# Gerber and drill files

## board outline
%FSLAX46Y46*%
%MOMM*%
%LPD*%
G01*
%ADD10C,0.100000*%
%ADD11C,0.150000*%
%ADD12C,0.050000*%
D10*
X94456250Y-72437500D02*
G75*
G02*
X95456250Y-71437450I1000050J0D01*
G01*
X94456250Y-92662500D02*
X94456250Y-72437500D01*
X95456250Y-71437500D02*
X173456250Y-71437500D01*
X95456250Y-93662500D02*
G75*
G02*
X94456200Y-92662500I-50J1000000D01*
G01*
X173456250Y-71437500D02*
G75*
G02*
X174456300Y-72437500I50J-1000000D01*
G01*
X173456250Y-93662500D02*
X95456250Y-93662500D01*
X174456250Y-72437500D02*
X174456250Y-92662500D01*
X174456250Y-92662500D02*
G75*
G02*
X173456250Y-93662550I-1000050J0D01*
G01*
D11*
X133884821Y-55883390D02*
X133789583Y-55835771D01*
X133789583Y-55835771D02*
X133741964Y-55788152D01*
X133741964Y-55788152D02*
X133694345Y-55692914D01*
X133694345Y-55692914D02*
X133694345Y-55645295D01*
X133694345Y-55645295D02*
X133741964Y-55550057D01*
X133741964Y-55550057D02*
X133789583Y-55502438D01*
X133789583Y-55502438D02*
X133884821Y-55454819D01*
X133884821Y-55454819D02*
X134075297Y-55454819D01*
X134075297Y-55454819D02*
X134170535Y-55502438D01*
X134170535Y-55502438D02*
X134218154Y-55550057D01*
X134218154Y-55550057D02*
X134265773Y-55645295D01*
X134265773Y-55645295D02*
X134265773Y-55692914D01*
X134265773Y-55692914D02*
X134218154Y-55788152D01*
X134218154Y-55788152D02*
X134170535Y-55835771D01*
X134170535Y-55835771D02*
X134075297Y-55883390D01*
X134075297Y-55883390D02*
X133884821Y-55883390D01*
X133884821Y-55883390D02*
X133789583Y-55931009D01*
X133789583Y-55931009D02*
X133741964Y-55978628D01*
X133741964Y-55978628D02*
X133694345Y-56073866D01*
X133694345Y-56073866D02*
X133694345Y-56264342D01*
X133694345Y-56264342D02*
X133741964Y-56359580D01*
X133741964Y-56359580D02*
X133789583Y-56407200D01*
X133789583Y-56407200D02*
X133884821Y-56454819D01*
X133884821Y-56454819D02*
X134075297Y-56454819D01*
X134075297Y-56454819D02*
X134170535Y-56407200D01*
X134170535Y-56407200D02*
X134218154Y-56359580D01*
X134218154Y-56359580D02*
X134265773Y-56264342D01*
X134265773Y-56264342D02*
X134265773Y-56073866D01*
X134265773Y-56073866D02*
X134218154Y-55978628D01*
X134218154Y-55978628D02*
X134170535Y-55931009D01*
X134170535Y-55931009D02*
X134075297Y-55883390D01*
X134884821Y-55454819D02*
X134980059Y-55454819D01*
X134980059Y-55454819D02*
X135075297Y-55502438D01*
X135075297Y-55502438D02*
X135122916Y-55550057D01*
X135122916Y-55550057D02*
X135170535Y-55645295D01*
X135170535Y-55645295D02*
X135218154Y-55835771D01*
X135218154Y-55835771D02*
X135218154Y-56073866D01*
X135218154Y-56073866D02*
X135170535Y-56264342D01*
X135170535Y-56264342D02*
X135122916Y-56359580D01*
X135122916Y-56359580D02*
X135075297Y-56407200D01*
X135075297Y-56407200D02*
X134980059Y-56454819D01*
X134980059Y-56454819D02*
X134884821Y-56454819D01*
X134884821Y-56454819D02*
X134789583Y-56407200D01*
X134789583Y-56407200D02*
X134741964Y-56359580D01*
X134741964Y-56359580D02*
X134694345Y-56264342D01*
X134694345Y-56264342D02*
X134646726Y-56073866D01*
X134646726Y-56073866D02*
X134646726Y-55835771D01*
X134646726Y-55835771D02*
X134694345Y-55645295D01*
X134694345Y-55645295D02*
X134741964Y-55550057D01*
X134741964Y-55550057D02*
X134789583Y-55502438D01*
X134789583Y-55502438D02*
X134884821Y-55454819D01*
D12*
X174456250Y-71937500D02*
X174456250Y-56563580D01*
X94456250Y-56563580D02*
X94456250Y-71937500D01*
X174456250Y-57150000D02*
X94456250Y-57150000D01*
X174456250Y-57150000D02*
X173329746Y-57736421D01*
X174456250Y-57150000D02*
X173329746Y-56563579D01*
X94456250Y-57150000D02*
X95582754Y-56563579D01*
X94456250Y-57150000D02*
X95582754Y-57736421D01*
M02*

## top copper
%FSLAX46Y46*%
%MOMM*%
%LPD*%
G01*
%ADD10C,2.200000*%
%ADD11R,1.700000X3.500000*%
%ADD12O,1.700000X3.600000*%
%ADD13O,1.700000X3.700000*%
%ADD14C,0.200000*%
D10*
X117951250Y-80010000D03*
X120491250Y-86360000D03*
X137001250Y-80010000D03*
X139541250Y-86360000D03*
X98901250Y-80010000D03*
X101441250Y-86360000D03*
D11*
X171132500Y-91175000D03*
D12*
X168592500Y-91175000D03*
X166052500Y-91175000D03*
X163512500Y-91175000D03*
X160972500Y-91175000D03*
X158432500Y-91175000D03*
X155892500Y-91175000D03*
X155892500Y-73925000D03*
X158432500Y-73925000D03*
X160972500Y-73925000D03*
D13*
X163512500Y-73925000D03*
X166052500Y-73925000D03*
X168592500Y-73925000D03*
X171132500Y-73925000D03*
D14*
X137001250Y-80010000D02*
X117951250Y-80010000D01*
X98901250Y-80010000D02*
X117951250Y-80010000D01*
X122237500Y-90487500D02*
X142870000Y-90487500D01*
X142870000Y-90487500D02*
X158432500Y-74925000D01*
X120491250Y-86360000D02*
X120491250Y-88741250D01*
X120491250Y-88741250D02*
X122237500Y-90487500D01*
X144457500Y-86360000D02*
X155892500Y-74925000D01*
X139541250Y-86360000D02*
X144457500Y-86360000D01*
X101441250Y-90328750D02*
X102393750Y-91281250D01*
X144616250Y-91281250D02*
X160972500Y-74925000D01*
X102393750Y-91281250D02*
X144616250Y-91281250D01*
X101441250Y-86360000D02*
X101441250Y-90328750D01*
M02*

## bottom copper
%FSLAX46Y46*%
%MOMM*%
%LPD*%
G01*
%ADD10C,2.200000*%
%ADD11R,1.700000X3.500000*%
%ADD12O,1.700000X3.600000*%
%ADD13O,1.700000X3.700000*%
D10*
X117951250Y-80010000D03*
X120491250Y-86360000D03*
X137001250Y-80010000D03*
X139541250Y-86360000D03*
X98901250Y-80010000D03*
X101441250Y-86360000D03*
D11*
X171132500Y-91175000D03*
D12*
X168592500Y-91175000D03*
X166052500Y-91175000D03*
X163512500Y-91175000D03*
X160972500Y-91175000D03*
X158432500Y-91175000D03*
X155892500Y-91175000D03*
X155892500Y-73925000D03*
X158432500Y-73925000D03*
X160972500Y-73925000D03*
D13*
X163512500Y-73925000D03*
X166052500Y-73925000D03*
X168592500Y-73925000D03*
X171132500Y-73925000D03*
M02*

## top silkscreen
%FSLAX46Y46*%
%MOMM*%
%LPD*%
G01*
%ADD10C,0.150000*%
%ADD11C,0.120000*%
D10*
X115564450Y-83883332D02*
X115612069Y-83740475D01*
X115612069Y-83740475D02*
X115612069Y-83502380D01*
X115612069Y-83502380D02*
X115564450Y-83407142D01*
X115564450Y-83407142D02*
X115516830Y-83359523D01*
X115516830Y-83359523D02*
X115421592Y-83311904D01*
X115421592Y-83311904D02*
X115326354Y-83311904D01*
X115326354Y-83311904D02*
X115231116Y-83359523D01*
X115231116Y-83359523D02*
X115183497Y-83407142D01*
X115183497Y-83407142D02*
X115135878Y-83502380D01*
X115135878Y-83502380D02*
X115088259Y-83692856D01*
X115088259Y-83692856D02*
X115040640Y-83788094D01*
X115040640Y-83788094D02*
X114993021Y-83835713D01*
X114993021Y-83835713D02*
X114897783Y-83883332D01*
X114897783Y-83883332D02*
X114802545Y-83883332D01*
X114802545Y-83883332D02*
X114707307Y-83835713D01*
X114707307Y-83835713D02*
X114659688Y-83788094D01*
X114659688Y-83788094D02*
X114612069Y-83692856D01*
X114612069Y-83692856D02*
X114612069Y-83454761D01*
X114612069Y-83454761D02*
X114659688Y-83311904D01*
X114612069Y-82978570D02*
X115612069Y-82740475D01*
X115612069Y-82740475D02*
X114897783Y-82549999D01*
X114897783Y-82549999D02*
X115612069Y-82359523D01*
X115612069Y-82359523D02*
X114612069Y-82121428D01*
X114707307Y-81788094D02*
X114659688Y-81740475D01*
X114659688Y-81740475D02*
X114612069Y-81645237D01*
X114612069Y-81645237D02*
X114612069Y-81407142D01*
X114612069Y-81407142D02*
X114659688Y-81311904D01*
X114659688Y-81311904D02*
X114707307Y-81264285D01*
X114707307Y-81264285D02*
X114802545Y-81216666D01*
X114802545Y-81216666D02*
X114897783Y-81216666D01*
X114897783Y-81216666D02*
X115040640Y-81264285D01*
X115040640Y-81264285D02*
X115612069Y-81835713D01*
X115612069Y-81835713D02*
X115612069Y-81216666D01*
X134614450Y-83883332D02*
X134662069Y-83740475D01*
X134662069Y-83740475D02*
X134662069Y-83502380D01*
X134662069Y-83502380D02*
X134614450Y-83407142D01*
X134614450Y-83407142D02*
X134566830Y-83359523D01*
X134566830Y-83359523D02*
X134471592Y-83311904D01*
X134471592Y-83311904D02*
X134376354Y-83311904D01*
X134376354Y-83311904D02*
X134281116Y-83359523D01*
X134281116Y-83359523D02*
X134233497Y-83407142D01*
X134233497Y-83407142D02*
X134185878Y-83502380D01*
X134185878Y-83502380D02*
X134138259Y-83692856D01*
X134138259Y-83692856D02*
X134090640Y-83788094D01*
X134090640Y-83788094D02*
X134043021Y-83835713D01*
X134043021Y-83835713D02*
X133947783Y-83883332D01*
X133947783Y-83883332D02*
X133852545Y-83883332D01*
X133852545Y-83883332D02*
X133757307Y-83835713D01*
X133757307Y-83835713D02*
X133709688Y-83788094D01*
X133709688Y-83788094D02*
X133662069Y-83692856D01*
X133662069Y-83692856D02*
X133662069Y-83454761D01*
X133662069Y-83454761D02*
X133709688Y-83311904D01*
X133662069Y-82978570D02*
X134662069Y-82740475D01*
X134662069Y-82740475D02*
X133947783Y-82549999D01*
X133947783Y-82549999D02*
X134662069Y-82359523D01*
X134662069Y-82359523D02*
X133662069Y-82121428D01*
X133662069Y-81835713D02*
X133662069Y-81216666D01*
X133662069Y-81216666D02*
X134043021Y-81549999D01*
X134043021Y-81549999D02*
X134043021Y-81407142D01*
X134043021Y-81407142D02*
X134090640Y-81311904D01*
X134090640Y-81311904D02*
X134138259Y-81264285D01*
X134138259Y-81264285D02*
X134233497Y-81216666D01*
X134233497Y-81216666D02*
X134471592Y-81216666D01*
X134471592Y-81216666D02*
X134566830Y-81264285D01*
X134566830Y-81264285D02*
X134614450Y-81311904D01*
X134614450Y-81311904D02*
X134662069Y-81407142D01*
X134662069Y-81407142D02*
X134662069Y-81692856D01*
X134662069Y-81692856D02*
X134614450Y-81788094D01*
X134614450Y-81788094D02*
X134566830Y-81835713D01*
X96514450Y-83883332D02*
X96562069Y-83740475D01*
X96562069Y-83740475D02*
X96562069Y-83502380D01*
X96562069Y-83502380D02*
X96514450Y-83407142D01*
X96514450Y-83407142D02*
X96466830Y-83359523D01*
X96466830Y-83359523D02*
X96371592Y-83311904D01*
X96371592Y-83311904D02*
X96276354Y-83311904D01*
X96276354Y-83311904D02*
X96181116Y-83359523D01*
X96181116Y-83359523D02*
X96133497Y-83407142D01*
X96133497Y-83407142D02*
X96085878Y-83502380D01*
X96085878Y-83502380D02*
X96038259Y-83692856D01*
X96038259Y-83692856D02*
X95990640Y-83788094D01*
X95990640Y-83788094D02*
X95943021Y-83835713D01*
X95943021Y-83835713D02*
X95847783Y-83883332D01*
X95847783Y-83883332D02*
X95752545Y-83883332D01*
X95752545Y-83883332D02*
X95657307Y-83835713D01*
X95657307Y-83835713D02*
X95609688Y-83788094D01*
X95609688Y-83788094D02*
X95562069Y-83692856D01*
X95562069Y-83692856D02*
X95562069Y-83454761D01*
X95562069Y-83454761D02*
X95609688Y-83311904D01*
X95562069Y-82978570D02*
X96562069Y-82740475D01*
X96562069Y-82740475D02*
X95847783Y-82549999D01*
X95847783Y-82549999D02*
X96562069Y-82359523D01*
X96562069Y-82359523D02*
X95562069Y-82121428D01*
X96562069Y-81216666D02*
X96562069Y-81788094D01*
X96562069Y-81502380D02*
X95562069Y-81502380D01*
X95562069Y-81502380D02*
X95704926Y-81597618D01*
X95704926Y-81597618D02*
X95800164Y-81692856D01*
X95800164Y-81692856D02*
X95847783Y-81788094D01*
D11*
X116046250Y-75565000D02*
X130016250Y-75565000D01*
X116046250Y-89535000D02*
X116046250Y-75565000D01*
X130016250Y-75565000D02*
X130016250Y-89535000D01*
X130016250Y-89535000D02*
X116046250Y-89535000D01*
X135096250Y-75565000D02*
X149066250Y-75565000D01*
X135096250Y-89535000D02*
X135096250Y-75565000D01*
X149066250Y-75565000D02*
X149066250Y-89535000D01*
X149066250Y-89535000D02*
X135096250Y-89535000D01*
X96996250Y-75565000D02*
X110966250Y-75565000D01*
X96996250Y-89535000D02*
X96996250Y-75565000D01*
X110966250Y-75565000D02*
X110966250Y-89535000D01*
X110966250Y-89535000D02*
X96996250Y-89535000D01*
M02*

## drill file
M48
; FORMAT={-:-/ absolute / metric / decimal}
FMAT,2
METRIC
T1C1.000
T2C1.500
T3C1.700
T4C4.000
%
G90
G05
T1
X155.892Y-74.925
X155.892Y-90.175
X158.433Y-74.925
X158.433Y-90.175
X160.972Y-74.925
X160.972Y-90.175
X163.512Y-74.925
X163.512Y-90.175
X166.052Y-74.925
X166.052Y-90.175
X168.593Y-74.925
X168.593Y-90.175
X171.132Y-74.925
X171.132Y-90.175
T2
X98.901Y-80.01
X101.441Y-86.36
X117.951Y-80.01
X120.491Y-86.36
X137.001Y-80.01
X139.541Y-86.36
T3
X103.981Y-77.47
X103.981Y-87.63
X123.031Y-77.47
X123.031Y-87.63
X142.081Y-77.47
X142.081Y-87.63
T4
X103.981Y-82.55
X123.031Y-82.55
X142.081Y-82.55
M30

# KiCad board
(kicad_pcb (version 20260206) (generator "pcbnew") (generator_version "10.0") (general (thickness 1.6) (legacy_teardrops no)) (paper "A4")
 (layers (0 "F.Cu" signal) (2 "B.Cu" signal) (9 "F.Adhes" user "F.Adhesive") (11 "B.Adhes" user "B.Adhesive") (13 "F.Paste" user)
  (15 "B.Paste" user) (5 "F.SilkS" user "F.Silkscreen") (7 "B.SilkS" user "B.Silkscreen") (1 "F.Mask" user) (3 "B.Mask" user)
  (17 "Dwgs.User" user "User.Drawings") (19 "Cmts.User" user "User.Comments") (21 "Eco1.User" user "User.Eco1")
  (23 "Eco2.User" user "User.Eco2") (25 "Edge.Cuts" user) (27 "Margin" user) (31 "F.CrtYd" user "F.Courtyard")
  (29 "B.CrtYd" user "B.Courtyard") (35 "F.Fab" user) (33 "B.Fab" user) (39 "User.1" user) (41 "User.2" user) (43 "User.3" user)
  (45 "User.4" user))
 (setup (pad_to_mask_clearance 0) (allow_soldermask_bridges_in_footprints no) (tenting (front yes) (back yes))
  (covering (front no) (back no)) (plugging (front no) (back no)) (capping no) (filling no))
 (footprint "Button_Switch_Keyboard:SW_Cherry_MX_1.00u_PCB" (layer "F.Cu") (at 117.95125 80.01 90)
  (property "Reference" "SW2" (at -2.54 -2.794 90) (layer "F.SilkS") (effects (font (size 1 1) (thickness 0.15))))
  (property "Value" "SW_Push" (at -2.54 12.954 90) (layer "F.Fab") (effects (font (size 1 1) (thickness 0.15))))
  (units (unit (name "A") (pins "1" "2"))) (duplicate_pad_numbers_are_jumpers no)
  (fp_line (start 4.445 -1.905) (end 4.445 12.065) (stroke (width 0.12) (type solid)) (layer "F.SilkS"))
  (fp_line (start -9.525 -1.905) (end 4.445 -1.905) (stroke (width 0.12) (type solid)) (layer "F.SilkS"))
  (fp_line (start 4.445 12.065) (end -9.525 12.065) (stroke (width 0.12) (type solid)) (layer "F.SilkS"))
  (fp_line (start -9.525 12.065) (end -9.525 -1.905) (stroke (width 0.12) (type solid)) (layer "F.SilkS"))
  (pad "" np_thru_hole circle (at -7.62 5.08 90) (size 1.7 1.7) (drill 1.7) (layers "*.Cu" "*.Mask"))
  (pad "" np_thru_hole circle (at -2.54 5.08 90) (size 4 4) (drill 4) (layers "*.Cu" "*.Mask"))
  (pad "" np_thru_hole circle (at 2.54 5.08 90) (size 1.7 1.7) (drill 1.7) (layers "*.Cu" "*.Mask"))
  (pad "1" thru_hole circle (at 0 0 90) (size 2.2 2.2) (drill 1.5) (layers "*.Cu" "*.Mask") (remove_unused_layers no) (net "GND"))
  (pad "2" thru_hole circle (at -6.35 2.54 90) (size 2.2 2.2) (drill 1.5) (layers "*.Cu" "*.Mask") (remove_unused_layers no)
   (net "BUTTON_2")))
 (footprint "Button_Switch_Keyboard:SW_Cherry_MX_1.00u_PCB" (layer "F.Cu") (at 137.00125 80.01 90)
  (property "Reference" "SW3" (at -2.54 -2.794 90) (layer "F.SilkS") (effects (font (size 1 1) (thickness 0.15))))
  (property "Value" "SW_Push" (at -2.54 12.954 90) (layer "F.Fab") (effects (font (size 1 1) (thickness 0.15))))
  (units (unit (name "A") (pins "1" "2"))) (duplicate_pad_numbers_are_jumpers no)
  (fp_line (start 4.445 -1.905) (end 4.445 12.065) (stroke (width 0.12) (type solid)) (layer "F.SilkS"))
  (fp_line (start -9.525 -1.905) (end 4.445 -1.905) (stroke (width 0.12) (type solid)) (layer "F.SilkS"))
  (fp_line (start 4.445 12.065) (end -9.525 12.065) (stroke (width 0.12) (type solid)) (layer "F.SilkS"))
  (fp_line (start -9.525 12.065) (end -9.525 -1.905) (stroke (width 0.12) (type solid)) (layer "F.SilkS"))
  (pad "" np_thru_hole circle (at -7.62 5.08 90) (size 1.7 1.7) (drill 1.7) (layers "*.Cu" "*.Mask"))
  (pad "" np_thru_hole circle (at -2.54 5.08 90) (size 4 4) (drill 4) (layers "*.Cu" "*.Mask"))
  (pad "" np_thru_hole circle (at 2.54 5.08 90) (size 1.7 1.7) (drill 1.7) (layers "*.Cu" "*.Mask"))
  (pad "1" thru_hole circle (at 0 0 90) (size 2.2 2.2) (drill 1.5) (layers "*.Cu" "*.Mask") (remove_unused_layers no) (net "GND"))
  (pad "2" thru_hole circle (at -6.35 2.54 90) (size 2.2 2.2) (drill 1.5) (layers "*.Cu" "*.Mask") (remove_unused_layers no)
   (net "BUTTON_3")))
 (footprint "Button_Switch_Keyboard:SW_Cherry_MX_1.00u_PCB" (layer "F.Cu") (at 98.90125 80.01 90)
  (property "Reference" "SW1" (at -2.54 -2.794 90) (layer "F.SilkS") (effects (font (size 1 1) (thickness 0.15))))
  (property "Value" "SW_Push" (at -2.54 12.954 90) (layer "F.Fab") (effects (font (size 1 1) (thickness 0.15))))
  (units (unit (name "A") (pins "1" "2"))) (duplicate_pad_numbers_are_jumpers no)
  (fp_line (start 4.445 -1.905) (end 4.445 12.065) (stroke (width 0.12) (type solid)) (layer "F.SilkS"))
  (fp_line (start -9.525 -1.905) (end 4.445 -1.905) (stroke (width 0.12) (type solid)) (layer "F.SilkS"))
  (fp_line (start 4.445 12.065) (end -9.525 12.065) (stroke (width 0.12) (type solid)) (layer "F.SilkS"))
  (fp_line (start -9.525 12.065) (end -9.525 -1.905) (stroke (width 0.12) (type solid)) (layer "F.SilkS"))
  (pad "" np_thru_hole circle (at -7.62 5.08 90) (size 1.7 1.7) (drill 1.7) (layers "*.Cu" "*.Mask"))
  (pad "" np_thru_hole circle (at -2.54 5.08 90) (size 4 4) (drill 4) (layers "*.Cu" "*.Mask"))
  (pad "" np_thru_hole circle (at 2.54 5.08 90) (size 1.7 1.7) (drill 1.7) (layers "*.Cu" "*.Mask"))
  (pad "1" thru_hole circle (at 0 0 90) (size 2.2 2.2) (drill 1.5) (layers "*.Cu" "*.Mask") (remove_unused_layers no) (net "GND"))
  (pad "2" thru_hole circle (at -6.35 2.54 90) (size 2.2 2.2) (drill 1.5) (layers "*.Cu" "*.Mask") (remove_unused_layers no)
   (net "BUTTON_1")))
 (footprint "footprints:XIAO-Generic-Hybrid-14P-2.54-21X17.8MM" (layer "B.Cu") (at 163.5125 82.55 90)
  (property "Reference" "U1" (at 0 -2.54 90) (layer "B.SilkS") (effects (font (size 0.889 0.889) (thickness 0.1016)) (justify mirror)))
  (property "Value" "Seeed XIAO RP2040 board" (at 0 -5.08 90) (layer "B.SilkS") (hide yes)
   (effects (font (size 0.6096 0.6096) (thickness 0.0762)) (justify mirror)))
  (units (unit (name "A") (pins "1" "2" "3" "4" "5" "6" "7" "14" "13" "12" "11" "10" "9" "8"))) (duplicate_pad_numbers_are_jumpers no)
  (pad "1" thru_hole rect (at -7.625 7.62 90) (size 3.5 1.7) (drill 1 (offset -1 0)) (layers "*.Cu" "*.Mask") (remove_unused_layers no)
   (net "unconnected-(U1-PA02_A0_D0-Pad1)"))
  (pad "2" thru_hole oval (at -7.625 5.08 90) (size 3.6 1.7) (drill 1 (offset -1 0)) (layers "*.Cu" "*.Mask") (remove_unused_layers no)
   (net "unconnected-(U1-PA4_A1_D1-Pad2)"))
  (pad "3" thru_hole oval (at -7.625 2.54 90) (size 3.6 1.7) (drill 1 (offset -1 0)) (layers "*.Cu" "*.Mask") (remove_unused_layers no)
   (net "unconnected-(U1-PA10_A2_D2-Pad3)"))
  (pad "4" thru_hole oval (at -7.625 0 90) (size 3.6 1.7) (drill 1 (offset -1 0)) (layers "*.Cu" "*.Mask") (remove_unused_layers no)
   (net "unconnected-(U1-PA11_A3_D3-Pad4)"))
  (pad "5" thru_hole oval (at -7.625 -2.54 90) (size 3.6 1.7) (drill 1 (offset -1 0)) (layers "*.Cu" "*.Mask") (remove_unused_layers no)
   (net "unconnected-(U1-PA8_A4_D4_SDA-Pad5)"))
  (pad "6" thru_hole oval (at -7.625 -5.08 270) (size 3.6 1.7) (drill 1 (offset 1 0)) (layers "*.Cu" "*.Mask") (remove_unused_layers no)
   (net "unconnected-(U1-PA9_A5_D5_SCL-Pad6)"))
  (pad "7" thru_hole oval (at -7.625 -7.62 90) (size 3.6 1.7) (drill 1 (offset -1 0)) (layers "*.Cu" "*.Mask") (remove_unused_layers no)
   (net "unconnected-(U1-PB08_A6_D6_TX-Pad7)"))
  (pad "8" thru_hole oval (at 7.625 -7.62 90) (size 3.6 1.7) (drill 1 (offset 1 0)) (layers "*.Cu" "*.Mask") (remove_unused_layers no)
   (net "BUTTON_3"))
  (pad "9" thru_hole oval (at 7.625 -5.08 90) (size 3.6 1.7) (drill 1 (offset 1 0)) (layers "*.Cu" "*.Mask") (remove_unused_layers no)
   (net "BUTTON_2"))
  (pad "10" thru_hole oval (at 7.625 -2.54 90) (size 3.6 1.7) (drill 1 (offset 1 0)) (layers "*.Cu" "*.Mask") (remove_unused_layers no)
   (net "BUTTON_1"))
  (pad "11" thru_hole oval (at 7.625 0 90) (size 3.7 1.7) (drill 1 (offset 1 0)) (layers "*.Cu" "*.Mask") (remove_unused_layers no)
   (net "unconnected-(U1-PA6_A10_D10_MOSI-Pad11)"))
  (pad "12" thru_hole oval (at 7.625 2.54 90) (size 3.7 1.7) (drill 1 (offset 1 0)) (layers "*.Cu" "*.Mask") (remove_unused_layers no)
   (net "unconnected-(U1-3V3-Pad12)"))
  (pad "13" thru_hole oval (at 7.625 5.08 90) (size 3.7 1.7) (drill 1 (offset 1 0)) (layers "*.Cu" "*.Mask") (remove_unused_layers no)
   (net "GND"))
  (pad "14" thru_hole oval (at 7.625 7.62 90) (size 3.7 1.7) (drill 1 (offset 1 0)) (layers "*.Cu" "*.Mask") (remove_unused_layers no)
   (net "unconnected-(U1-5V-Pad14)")))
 (gr_arc (start 94.45625 72.4375) (mid 94.749146 71.730411) (end 95.45625 71.4375) (stroke (width 0.1) (type default)) (layer "Edge.Cuts"))
 (gr_line (start 94.45625 92.6625) (end 94.45625 72.4375) (stroke (width 0.1) (type default)) (layer "Edge.Cuts"))
 (gr_line (start 95.45625 71.4375) (end 173.45625 71.4375) (stroke (width 0.1) (type default)) (layer "Edge.Cuts"))
 (gr_arc (start 95.45625 93.6625) (mid 94.749143 93.369607) (end 94.45625 92.6625) (stroke (width 0.1) (type default)) (layer "Edge.Cuts"))
 (gr_arc (start 173.45625 71.4375) (mid 174.163357 71.730393) (end 174.45625 72.4375) (stroke (width 0.1) (type default))
  (layer "Edge.Cuts"))
 (gr_line (start 173.45625 93.6625) (end 95.45625 93.6625) (stroke (width 0.1) (type default)) (layer "Edge.Cuts"))
 (gr_line (start 174.45625 72.4375) (end 174.45625 92.6625) (stroke (width 0.1) (type default)) (layer "Edge.Cuts"))
 (gr_arc (start 174.45625 92.6625) (mid 174.163354 93.369589) (end 173.45625 93.6625) (stroke (width 0.1) (type default))
  (layer "Edge.Cuts"))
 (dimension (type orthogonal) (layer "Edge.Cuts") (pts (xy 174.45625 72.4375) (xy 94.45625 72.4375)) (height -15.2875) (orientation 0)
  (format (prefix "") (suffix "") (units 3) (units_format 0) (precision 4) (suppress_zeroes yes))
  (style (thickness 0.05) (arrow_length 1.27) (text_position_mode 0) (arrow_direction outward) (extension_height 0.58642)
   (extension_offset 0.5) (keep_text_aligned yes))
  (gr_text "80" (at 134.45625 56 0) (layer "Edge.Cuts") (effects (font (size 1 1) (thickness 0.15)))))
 (segment (start 137.00125 80.01) (end 117.95125 80.01) (width 0.2) (layer "F.Cu") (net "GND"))
 (segment (start 98.90125 80.01) (end 117.95125 80.01) (width 0.2) (layer "F.Cu") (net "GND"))
 (segment (start 122.2375 90.4875) (end 142.87 90.4875) (width 0.2) (layer "F.Cu") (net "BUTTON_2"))
 (segment (start 142.87 90.4875) (end 158.4325 74.925) (width 0.2) (layer "F.Cu") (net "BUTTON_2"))
 (segment (start 120.49125 86.36) (end 120.49125 88.74125) (width 0.2) (layer "F.Cu") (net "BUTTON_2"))
 (segment (start 120.49125 88.74125) (end 122.2375 90.4875) (width 0.2) (layer "F.Cu") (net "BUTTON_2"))
 (segment (start 144.4575 86.36) (end 155.8925 74.925) (width 0.2) (layer "F.Cu") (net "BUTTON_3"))
 (segment (start 139.54125 86.36) (end 144.4575 86.36) (width 0.2) (layer "F.Cu") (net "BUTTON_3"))
 (segment (start 101.44125 90.32875) (end 102.39375 91.28125) (width 0.2) (layer "F.Cu") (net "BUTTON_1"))
 (segment (start 144.61625 91.28125) (end 160.9725 74.925) (width 0.2) (layer "F.Cu") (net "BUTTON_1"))
 (segment (start 102.39375 91.28125) (end 144.61625 91.28125) (width 0.2) (layer "F.Cu") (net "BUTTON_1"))
 (segment (start 101.44125 86.36) (end 101.44125 90.32875) (width 0.2) (layer "F.Cu") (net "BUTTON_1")))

